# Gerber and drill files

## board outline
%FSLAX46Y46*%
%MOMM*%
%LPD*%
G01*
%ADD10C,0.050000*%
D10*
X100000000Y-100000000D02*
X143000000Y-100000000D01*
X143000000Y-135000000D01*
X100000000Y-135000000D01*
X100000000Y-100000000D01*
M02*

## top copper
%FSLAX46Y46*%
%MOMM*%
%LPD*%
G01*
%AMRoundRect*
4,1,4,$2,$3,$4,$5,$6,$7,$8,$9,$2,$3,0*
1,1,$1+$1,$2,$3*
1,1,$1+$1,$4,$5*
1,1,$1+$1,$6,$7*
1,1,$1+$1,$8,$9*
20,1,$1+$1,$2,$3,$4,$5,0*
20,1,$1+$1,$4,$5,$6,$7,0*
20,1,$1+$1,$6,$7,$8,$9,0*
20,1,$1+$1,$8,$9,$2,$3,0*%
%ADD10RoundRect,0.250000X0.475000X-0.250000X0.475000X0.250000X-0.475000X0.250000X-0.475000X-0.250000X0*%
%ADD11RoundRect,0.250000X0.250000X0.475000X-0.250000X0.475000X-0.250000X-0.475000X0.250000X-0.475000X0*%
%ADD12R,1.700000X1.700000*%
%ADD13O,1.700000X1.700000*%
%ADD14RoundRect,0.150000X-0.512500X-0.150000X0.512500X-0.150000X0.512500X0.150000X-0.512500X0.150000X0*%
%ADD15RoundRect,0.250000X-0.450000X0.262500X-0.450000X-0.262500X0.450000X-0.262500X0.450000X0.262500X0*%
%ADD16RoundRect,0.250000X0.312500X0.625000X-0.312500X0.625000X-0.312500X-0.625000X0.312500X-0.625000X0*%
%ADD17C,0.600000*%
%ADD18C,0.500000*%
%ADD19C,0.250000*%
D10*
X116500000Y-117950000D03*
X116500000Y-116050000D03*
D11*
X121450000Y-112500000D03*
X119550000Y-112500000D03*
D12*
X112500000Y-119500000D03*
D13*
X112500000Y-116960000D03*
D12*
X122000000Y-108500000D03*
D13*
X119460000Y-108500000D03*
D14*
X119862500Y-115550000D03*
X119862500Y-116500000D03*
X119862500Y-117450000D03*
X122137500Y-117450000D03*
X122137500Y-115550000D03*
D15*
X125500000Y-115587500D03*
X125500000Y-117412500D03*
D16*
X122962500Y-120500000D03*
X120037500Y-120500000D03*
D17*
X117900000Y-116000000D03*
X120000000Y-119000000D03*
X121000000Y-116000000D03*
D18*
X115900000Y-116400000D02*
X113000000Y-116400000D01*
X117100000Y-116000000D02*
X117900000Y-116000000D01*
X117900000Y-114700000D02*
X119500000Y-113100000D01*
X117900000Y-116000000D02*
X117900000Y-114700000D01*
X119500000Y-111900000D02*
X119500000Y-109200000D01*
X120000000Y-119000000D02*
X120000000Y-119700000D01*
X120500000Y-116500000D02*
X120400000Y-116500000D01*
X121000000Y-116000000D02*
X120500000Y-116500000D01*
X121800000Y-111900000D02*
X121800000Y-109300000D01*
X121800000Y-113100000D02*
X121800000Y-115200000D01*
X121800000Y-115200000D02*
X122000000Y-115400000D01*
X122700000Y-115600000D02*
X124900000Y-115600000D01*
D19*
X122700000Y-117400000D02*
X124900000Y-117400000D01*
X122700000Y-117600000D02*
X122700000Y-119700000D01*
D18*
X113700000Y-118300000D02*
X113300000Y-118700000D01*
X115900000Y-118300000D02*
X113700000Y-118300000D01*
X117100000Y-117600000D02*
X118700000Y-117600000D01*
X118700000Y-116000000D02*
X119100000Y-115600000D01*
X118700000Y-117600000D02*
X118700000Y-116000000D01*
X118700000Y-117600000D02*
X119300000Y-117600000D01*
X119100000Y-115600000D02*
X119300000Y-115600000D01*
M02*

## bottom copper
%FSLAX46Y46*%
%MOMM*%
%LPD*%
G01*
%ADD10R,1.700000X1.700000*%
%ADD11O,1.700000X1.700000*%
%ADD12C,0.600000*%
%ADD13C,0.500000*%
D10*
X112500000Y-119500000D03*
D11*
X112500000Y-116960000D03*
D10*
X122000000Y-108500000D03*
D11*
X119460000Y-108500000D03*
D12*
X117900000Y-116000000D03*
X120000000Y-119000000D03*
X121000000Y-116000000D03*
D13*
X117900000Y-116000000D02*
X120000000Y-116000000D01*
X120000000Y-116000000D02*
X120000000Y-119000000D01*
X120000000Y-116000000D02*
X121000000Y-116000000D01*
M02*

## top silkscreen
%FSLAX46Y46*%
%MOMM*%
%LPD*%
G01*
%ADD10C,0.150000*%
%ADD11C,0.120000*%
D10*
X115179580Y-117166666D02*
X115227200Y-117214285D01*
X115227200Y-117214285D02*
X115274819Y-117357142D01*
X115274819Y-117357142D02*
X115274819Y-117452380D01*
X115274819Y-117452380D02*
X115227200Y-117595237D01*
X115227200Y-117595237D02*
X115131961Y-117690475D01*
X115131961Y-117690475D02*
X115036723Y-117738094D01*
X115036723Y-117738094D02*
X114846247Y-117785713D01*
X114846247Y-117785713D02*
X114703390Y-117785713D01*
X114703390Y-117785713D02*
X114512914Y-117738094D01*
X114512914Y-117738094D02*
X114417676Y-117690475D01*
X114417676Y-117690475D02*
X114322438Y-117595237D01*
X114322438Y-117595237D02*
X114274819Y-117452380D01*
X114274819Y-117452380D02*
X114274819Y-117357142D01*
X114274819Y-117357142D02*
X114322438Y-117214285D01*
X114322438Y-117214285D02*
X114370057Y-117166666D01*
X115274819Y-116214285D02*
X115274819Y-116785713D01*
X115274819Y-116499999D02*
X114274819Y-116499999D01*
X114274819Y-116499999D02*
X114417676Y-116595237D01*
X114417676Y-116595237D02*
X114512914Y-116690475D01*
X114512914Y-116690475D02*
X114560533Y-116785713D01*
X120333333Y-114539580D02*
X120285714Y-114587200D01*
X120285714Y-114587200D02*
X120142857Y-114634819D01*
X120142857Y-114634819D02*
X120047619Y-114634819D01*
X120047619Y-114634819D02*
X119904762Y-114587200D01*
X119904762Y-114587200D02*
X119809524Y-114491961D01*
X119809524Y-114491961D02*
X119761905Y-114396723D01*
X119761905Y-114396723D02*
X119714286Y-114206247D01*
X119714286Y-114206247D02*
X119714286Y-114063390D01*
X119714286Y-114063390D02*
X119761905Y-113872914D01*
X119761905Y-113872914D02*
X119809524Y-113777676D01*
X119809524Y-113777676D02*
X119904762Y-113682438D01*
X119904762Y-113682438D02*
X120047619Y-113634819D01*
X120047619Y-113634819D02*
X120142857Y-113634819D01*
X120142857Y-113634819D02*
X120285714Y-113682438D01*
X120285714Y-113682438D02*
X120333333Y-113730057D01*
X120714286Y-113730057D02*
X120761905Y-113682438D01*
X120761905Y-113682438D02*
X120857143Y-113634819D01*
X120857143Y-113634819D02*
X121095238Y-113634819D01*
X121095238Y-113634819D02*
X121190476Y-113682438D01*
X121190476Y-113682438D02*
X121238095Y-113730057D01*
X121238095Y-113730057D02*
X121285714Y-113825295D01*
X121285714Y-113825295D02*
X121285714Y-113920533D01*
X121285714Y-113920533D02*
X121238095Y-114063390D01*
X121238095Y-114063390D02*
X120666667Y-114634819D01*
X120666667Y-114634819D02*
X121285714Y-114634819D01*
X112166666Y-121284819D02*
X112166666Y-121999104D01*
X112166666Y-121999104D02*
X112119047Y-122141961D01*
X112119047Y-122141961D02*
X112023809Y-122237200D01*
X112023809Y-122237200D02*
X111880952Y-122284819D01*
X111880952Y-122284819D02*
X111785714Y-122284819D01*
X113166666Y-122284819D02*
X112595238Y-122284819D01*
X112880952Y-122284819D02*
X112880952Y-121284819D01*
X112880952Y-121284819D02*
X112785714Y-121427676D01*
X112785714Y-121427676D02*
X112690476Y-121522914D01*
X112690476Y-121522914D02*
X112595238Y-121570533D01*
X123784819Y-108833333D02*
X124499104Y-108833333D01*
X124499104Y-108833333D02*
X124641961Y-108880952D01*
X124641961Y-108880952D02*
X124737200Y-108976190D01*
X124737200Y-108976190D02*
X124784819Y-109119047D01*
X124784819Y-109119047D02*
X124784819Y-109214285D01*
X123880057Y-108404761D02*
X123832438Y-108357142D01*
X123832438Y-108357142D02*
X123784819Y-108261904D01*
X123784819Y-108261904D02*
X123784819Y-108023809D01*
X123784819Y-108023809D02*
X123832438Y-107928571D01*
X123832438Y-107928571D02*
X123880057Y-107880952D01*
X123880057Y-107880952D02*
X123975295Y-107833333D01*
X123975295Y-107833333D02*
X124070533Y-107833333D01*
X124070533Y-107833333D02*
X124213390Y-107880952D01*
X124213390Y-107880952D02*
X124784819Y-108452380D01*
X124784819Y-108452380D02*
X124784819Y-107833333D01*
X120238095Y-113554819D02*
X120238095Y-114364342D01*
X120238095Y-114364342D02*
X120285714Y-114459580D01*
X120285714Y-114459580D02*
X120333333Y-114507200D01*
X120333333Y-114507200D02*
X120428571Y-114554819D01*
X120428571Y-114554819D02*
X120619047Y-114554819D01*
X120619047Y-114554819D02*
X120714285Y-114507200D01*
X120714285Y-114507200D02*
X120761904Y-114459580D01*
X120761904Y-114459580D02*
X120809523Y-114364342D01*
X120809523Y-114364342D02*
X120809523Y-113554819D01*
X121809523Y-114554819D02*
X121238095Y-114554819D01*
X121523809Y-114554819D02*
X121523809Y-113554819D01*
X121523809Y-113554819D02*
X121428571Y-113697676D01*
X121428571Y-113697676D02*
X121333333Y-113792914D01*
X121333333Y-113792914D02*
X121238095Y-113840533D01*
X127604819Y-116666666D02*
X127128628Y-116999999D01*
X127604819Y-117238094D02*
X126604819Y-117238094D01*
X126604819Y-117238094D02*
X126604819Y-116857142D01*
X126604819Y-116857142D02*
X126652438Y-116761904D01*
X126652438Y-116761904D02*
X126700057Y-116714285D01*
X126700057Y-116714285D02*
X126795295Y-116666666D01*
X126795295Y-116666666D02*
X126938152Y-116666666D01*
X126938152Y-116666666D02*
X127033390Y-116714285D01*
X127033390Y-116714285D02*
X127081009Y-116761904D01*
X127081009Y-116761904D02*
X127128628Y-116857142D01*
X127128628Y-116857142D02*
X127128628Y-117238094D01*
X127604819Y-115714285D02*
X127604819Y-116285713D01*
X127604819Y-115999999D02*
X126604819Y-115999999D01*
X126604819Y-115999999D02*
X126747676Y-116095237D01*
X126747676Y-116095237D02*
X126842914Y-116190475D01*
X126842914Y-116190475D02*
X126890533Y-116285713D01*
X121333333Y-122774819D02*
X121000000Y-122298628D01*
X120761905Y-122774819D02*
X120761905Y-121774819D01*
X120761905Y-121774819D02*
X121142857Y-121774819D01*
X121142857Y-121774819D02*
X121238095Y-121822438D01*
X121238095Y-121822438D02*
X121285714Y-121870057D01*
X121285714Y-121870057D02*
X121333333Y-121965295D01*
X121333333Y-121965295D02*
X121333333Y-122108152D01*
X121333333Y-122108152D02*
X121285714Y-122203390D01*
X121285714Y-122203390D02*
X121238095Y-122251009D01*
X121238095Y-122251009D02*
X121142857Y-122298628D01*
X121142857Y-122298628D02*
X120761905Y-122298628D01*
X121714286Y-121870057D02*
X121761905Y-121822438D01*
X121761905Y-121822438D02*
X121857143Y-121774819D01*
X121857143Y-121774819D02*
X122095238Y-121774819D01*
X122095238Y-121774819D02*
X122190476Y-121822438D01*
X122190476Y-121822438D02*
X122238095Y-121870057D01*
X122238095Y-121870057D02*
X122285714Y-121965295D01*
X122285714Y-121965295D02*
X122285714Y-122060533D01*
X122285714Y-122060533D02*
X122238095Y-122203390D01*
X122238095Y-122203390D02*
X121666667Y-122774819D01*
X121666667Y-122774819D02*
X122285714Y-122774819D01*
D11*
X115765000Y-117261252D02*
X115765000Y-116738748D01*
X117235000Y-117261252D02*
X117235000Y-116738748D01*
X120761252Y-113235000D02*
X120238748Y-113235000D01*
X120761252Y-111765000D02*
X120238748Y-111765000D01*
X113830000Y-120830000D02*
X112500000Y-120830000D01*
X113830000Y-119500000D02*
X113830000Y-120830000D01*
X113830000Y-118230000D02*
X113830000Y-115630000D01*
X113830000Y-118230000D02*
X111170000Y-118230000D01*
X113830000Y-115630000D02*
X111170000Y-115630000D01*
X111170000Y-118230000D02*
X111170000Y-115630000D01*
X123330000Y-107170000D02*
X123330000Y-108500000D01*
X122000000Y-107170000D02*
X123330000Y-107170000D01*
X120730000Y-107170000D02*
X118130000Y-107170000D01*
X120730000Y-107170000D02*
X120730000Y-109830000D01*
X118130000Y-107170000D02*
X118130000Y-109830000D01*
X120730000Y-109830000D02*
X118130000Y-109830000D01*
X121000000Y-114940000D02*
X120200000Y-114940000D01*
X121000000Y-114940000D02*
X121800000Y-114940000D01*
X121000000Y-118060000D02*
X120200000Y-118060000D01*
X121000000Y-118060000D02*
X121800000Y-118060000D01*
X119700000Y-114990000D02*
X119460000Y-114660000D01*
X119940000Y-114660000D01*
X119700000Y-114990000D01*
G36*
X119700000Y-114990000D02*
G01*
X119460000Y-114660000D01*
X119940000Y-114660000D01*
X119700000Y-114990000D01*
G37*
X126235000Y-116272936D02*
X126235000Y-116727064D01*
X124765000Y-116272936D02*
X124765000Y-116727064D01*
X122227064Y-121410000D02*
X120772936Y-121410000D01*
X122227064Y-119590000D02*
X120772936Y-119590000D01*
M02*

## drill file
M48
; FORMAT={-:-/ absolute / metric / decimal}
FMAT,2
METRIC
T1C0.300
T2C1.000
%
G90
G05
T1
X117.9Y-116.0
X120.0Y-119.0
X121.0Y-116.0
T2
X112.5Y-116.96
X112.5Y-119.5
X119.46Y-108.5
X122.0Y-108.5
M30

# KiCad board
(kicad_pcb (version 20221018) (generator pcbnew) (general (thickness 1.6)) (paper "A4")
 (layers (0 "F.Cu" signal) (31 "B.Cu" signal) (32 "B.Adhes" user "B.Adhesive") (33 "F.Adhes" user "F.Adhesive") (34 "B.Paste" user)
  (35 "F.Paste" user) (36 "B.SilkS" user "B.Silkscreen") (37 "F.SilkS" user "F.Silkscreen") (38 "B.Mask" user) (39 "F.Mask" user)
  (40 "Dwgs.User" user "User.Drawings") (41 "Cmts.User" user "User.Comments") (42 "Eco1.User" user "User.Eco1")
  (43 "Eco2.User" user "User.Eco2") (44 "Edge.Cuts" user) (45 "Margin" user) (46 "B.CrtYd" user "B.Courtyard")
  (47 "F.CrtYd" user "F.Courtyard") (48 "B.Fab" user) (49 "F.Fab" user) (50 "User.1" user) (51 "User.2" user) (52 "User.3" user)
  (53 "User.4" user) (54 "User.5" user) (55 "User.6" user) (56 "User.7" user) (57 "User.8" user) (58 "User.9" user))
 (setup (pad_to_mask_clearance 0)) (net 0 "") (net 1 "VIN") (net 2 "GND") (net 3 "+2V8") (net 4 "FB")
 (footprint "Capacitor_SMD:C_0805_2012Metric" (layer "F.Cu") (at 116.5 117 90)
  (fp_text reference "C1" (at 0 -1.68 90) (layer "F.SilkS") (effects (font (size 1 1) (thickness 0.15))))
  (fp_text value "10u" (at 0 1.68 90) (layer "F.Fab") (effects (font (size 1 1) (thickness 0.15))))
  (fp_line (start -0.261252 -0.735) (end 0.261252 -0.735) (stroke (width 0.12) (type solid)) (layer "F.SilkS"))
  (fp_line (start -0.261252 0.735) (end 0.261252 0.735) (stroke (width 0.12) (type solid)) (layer "F.SilkS"))
  (pad "1" smd roundrect (at -0.95 0 90) (size 1 1.45) (layers "F.Cu" "F.Paste" "F.Mask") (roundrect_rratio 0.25) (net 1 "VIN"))
  (pad "2" smd roundrect (at 0.95 0 90) (size 1 1.45) (layers "F.Cu" "F.Paste" "F.Mask") (roundrect_rratio 0.25) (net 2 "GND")))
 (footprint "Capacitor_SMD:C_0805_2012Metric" (layer "F.Cu") (at 120.5 112.5 180)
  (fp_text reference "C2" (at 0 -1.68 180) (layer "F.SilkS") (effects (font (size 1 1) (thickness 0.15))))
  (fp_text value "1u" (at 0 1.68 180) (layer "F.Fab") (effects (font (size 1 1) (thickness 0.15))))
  (fp_line (start -0.261252 -0.735) (end 0.261252 -0.735) (stroke (width 0.12) (type solid)) (layer "F.SilkS"))
  (fp_line (start -0.261252 0.735) (end 0.261252 0.735) (stroke (width 0.12) (type solid)) (layer "F.SilkS"))
  (pad "1" smd roundrect (at -0.95 0 180) (size 1 1.45) (layers "F.Cu" "F.Paste" "F.Mask") (roundrect_rratio 0.25) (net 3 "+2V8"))
  (pad "2" smd roundrect (at 0.95 0 180) (size 1 1.45) (layers "F.Cu" "F.Paste" "F.Mask") (roundrect_rratio 0.25) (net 2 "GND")))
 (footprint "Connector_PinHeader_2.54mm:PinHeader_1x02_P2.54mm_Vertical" (layer "F.Cu") (at 112.5 119.5 180)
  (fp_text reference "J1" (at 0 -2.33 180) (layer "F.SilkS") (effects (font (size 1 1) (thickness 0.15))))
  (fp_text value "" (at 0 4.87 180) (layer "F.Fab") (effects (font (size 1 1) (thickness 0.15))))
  (fp_line (start -1.33 -1.33) (end 0 -1.33) (stroke (width 0.12) (type solid)) (layer "F.SilkS"))
  (fp_line (start -1.33 0) (end -1.33 -1.33) (stroke (width 0.12) (type solid)) (layer "F.SilkS"))
  (fp_line (start -1.33 1.27) (end -1.33 3.87) (stroke (width 0.12) (type solid)) (layer "F.SilkS"))
  (fp_line (start -1.33 1.27) (end 1.33 1.27) (stroke (width 0.12) (type solid)) (layer "F.SilkS"))
  (fp_line (start -1.33 3.87) (end 1.33 3.87) (stroke (width 0.12) (type solid)) (layer "F.SilkS"))
  (fp_line (start 1.33 1.27) (end 1.33 3.87) (stroke (width 0.12) (type solid)) (layer "F.SilkS"))
  (pad "1" thru_hole rect (at 0 0 180) (size 1.7 1.7) (drill 1) (layers "*.Cu" "*.Mask") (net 1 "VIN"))
  (pad "2" thru_hole oval (at 0 2.54 180) (size 1.7 1.7) (drill 1) (layers "*.Cu" "*.Mask") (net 2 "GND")))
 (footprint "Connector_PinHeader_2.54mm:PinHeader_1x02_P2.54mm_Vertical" (layer "F.Cu") (at 122 108.5 -90)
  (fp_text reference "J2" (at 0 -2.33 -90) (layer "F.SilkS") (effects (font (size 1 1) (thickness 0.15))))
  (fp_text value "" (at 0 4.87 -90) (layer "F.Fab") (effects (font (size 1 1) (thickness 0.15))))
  (fp_line (start -1.33 -1.33) (end 0 -1.33) (stroke (width 0.12) (type solid)) (layer "F.SilkS"))
  (fp_line (start -1.33 0) (end -1.33 -1.33) (stroke (width 0.12) (type solid)) (layer "F.SilkS"))
  (fp_line (start -1.33 1.27) (end -1.33 3.87) (stroke (width 0.12) (type solid)) (layer "F.SilkS"))
  (fp_line (start -1.33 1.27) (end 1.33 1.27) (stroke (width 0.12) (type solid)) (layer "F.SilkS"))
  (fp_line (start -1.33 3.87) (end 1.33 3.87) (stroke (width 0.12) (type solid)) (layer "F.SilkS"))
  (fp_line (start 1.33 1.27) (end 1.33 3.87) (stroke (width 0.12) (type solid)) (layer "F.SilkS"))
  (pad "1" thru_hole rect (at 0 0 270) (size 1.7 1.7) (drill 1) (layers "*.Cu" "*.Mask") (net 3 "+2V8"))
  (pad "2" thru_hole oval (at 0 2.54 270) (size 1.7 1.7) (drill 1) (layers "*.Cu" "*.Mask") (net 2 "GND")))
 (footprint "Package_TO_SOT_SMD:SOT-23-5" (layer "F.Cu") (at 121 116.5)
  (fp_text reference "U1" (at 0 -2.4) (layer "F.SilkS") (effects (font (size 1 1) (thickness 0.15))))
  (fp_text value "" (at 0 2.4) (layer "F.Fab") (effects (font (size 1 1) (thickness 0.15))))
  (fp_line (start 0 -1.56) (end -0.8 -1.56) (stroke (width 0.12) (type solid)) (layer "F.SilkS"))
  (fp_line (start 0 -1.56) (end 0.8 -1.56) (stroke (width 0.12) (type solid)) (layer "F.SilkS"))
  (fp_line (start 0 1.56) (end -0.8 1.56) (stroke (width 0.12) (type solid)) (layer "F.SilkS"))
  (fp_line (start 0 1.56) (end 0.8 1.56) (stroke (width 0.12) (type solid)) (layer "F.SilkS"))
  (fp_poly
   (pts (xy -1.3 -1.51) (xy -1.54 -1.84) (xy -1.06 -1.84) (xy -1.3 -1.51)) (stroke (width 0.12) (type solid)) (fill solid) (layer "F.SilkS"))
  (pad "1" smd roundrect (at -1.1375 -0.95) (size 1.325 0.6) (layers "F.Cu" "F.Paste" "F.Mask") (roundrect_rratio 0.25) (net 1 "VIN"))
  (pad "2" smd roundrect (at -1.1375 0) (size 1.325 0.6) (layers "F.Cu" "F.Paste" "F.Mask") (roundrect_rratio 0.25) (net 2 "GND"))
  (pad "3" smd roundrect (at -1.1375 0.95) (size 1.325 0.6) (layers "F.Cu" "F.Paste" "F.Mask") (roundrect_rratio 0.25) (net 1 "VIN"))
  (pad "4" smd roundrect (at 1.1375 0.95) (size 1.325 0.6) (layers "F.Cu" "F.Paste" "F.Mask") (roundrect_rratio 0.25) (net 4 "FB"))
  (pad "5" smd roundrect (at 1.1375 -0.95) (size 1.325 0.6) (layers "F.Cu" "F.Paste" "F.Mask") (roundrect_rratio 0.25) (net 3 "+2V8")))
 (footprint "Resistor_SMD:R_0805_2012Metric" (layer "F.Cu") (at 125.5 116.5 -90)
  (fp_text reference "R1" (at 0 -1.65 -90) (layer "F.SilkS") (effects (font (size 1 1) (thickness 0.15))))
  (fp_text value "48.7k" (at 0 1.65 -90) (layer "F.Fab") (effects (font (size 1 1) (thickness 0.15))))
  (fp_line (start -0.227064 -0.735) (end 0.227064 -0.735) (stroke (width 0.12) (type solid)) (layer "F.SilkS"))
  (fp_line (start -0.227064 0.735) (end 0.227064 0.735) (stroke (width 0.12) (type solid)) (layer "F.SilkS"))
  (pad "1" smd roundrect (at -0.9125 0 270) (size 1.025 1.4) (layers "F.Cu" "F.Paste" "F.Mask") (roundrect_rratio 0.243902) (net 3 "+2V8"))
  (pad "2" smd roundrect (at 0.9125 0 270) (size 1.025 1.4) (layers "F.Cu" "F.Paste" "F.Mask") (roundrect_rratio 0.243902) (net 4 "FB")))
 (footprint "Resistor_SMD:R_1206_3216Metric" (layer "F.Cu") (at 121.5 120.5 180)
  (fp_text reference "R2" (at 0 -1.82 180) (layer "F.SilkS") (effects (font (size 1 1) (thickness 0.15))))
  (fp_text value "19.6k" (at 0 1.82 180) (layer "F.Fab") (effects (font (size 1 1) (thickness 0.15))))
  (fp_line (start -0.727064 -0.91) (end 0.727064 -0.91) (stroke (width 0.12) (type solid)) (layer "F.SilkS"))
  (fp_line (start -0.727064 0.91) (end 0.727064 0.91) (stroke (width 0.12) (type solid)) (layer "F.SilkS"))
  (pad "1" smd roundrect (at -1.4625 0 180) (size 1.125 1.75) (layers "F.Cu" "F.Paste" "F.Mask") (roundrect_rratio 0.222222) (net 4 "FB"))
  (pad "2" smd roundrect (at 1.4625 0 180) (size 1.125 1.75) (layers "F.Cu" "F.Paste" "F.Mask") (roundrect_rratio 0.222222) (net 2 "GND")))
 (gr_rect (start 100 100) (end 143 135) (stroke (width 0.05) (type default)) (fill none) (layer "Edge.Cuts"))
 (segment (start 115.9 116.4) (end 113 116.4) (width 0.5) (layer "F.Cu") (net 2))
 (segment (start 117.1 116) (end 117.9 116) (width 0.5) (layer "F.Cu") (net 2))
 (segment (start 117.9 114.7) (end 119.5 113.1) (width 0.5) (layer "F.Cu") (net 2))
 (segment (start 117.9 116) (end 117.9 114.7) (width 0.5) (layer "F.Cu") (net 2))
 (segment (start 119.5 111.9) (end 119.5 109.2) (width 0.5) (layer "F.Cu") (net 2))
 (segment (start 120 119) (end 120 119.7) (width 0.5) (layer "F.Cu") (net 2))
 (segment (start 120.5 116.5) (end 120.4 116.5) (width 0.5) (layer "F.Cu") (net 2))
 (segment (start 121 116) (end 120.5 116.5) (width 0.5) (layer "F.Cu") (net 2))
 (segment (start 121.8 111.9) (end 121.8 109.3) (width 0.5) (layer "F.Cu") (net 3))
 (segment (start 121.8 113.1) (end 121.8 115.2) (width 0.5) (layer "F.Cu") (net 3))
 (segment (start 121.8 115.2) (end 122 115.4) (width 0.5) (layer "F.Cu") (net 3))
 (segment (start 122.7 115.6) (end 124.9 115.6) (width 0.5) (layer "F.Cu") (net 3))
 (segment (start 122.7 117.4) (end 124.9 117.4) (width 0.25) (layer "F.Cu") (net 4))
 (segment (start 122.7 117.6) (end 122.7 119.7) (width 0.25) (layer "F.Cu") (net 4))
 (via (at 117.9 116) (size 0.6) (drill 0.3) (layers "F.Cu" "B.Cu") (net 2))
 (via (at 120 119) (size 0.6) (drill 0.3) (layers "F.Cu" "B.Cu") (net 2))
 (via (at 121 116) (size 0.6) (drill 0.3) (layers "F.Cu" "B.Cu") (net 2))
 (segment (start 113.7 118.3) (end 113.3 118.7) (width 0.5) (layer "F.Cu") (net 1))
 (segment (start 115.9 118.3) (end 113.7 118.3) (width 0.5) (layer "F.Cu") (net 1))
 (segment (start 117.1 117.6) (end 118.7 117.6) (width 0.5) (layer "F.Cu") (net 1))
 (segment (start 117.9 116) (end 120 116) (width 0.5) (layer "B.Cu") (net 2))
 (segment (start 118.7 116) (end 119.1 115.6) (width 0.5) (layer "F.Cu") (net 1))
 (segment (start 118.7 117.6) (end 118.7 116) (width 0.5) (layer "F.Cu") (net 1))
 (segment (start 118.7 117.6) (end 119.3 117.6) (width 0.5) (layer "F.Cu") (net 1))
 (segment (start 119.1 115.6) (end 119.3 115.6) (width 0.5) (layer "F.Cu") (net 1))
 (segment (start 120 116) (end 120 119) (width 0.5) (layer "B.Cu") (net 2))
 (segment (start 120 116) (end 121 116) (width 0.5) (layer "B.Cu") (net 2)))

